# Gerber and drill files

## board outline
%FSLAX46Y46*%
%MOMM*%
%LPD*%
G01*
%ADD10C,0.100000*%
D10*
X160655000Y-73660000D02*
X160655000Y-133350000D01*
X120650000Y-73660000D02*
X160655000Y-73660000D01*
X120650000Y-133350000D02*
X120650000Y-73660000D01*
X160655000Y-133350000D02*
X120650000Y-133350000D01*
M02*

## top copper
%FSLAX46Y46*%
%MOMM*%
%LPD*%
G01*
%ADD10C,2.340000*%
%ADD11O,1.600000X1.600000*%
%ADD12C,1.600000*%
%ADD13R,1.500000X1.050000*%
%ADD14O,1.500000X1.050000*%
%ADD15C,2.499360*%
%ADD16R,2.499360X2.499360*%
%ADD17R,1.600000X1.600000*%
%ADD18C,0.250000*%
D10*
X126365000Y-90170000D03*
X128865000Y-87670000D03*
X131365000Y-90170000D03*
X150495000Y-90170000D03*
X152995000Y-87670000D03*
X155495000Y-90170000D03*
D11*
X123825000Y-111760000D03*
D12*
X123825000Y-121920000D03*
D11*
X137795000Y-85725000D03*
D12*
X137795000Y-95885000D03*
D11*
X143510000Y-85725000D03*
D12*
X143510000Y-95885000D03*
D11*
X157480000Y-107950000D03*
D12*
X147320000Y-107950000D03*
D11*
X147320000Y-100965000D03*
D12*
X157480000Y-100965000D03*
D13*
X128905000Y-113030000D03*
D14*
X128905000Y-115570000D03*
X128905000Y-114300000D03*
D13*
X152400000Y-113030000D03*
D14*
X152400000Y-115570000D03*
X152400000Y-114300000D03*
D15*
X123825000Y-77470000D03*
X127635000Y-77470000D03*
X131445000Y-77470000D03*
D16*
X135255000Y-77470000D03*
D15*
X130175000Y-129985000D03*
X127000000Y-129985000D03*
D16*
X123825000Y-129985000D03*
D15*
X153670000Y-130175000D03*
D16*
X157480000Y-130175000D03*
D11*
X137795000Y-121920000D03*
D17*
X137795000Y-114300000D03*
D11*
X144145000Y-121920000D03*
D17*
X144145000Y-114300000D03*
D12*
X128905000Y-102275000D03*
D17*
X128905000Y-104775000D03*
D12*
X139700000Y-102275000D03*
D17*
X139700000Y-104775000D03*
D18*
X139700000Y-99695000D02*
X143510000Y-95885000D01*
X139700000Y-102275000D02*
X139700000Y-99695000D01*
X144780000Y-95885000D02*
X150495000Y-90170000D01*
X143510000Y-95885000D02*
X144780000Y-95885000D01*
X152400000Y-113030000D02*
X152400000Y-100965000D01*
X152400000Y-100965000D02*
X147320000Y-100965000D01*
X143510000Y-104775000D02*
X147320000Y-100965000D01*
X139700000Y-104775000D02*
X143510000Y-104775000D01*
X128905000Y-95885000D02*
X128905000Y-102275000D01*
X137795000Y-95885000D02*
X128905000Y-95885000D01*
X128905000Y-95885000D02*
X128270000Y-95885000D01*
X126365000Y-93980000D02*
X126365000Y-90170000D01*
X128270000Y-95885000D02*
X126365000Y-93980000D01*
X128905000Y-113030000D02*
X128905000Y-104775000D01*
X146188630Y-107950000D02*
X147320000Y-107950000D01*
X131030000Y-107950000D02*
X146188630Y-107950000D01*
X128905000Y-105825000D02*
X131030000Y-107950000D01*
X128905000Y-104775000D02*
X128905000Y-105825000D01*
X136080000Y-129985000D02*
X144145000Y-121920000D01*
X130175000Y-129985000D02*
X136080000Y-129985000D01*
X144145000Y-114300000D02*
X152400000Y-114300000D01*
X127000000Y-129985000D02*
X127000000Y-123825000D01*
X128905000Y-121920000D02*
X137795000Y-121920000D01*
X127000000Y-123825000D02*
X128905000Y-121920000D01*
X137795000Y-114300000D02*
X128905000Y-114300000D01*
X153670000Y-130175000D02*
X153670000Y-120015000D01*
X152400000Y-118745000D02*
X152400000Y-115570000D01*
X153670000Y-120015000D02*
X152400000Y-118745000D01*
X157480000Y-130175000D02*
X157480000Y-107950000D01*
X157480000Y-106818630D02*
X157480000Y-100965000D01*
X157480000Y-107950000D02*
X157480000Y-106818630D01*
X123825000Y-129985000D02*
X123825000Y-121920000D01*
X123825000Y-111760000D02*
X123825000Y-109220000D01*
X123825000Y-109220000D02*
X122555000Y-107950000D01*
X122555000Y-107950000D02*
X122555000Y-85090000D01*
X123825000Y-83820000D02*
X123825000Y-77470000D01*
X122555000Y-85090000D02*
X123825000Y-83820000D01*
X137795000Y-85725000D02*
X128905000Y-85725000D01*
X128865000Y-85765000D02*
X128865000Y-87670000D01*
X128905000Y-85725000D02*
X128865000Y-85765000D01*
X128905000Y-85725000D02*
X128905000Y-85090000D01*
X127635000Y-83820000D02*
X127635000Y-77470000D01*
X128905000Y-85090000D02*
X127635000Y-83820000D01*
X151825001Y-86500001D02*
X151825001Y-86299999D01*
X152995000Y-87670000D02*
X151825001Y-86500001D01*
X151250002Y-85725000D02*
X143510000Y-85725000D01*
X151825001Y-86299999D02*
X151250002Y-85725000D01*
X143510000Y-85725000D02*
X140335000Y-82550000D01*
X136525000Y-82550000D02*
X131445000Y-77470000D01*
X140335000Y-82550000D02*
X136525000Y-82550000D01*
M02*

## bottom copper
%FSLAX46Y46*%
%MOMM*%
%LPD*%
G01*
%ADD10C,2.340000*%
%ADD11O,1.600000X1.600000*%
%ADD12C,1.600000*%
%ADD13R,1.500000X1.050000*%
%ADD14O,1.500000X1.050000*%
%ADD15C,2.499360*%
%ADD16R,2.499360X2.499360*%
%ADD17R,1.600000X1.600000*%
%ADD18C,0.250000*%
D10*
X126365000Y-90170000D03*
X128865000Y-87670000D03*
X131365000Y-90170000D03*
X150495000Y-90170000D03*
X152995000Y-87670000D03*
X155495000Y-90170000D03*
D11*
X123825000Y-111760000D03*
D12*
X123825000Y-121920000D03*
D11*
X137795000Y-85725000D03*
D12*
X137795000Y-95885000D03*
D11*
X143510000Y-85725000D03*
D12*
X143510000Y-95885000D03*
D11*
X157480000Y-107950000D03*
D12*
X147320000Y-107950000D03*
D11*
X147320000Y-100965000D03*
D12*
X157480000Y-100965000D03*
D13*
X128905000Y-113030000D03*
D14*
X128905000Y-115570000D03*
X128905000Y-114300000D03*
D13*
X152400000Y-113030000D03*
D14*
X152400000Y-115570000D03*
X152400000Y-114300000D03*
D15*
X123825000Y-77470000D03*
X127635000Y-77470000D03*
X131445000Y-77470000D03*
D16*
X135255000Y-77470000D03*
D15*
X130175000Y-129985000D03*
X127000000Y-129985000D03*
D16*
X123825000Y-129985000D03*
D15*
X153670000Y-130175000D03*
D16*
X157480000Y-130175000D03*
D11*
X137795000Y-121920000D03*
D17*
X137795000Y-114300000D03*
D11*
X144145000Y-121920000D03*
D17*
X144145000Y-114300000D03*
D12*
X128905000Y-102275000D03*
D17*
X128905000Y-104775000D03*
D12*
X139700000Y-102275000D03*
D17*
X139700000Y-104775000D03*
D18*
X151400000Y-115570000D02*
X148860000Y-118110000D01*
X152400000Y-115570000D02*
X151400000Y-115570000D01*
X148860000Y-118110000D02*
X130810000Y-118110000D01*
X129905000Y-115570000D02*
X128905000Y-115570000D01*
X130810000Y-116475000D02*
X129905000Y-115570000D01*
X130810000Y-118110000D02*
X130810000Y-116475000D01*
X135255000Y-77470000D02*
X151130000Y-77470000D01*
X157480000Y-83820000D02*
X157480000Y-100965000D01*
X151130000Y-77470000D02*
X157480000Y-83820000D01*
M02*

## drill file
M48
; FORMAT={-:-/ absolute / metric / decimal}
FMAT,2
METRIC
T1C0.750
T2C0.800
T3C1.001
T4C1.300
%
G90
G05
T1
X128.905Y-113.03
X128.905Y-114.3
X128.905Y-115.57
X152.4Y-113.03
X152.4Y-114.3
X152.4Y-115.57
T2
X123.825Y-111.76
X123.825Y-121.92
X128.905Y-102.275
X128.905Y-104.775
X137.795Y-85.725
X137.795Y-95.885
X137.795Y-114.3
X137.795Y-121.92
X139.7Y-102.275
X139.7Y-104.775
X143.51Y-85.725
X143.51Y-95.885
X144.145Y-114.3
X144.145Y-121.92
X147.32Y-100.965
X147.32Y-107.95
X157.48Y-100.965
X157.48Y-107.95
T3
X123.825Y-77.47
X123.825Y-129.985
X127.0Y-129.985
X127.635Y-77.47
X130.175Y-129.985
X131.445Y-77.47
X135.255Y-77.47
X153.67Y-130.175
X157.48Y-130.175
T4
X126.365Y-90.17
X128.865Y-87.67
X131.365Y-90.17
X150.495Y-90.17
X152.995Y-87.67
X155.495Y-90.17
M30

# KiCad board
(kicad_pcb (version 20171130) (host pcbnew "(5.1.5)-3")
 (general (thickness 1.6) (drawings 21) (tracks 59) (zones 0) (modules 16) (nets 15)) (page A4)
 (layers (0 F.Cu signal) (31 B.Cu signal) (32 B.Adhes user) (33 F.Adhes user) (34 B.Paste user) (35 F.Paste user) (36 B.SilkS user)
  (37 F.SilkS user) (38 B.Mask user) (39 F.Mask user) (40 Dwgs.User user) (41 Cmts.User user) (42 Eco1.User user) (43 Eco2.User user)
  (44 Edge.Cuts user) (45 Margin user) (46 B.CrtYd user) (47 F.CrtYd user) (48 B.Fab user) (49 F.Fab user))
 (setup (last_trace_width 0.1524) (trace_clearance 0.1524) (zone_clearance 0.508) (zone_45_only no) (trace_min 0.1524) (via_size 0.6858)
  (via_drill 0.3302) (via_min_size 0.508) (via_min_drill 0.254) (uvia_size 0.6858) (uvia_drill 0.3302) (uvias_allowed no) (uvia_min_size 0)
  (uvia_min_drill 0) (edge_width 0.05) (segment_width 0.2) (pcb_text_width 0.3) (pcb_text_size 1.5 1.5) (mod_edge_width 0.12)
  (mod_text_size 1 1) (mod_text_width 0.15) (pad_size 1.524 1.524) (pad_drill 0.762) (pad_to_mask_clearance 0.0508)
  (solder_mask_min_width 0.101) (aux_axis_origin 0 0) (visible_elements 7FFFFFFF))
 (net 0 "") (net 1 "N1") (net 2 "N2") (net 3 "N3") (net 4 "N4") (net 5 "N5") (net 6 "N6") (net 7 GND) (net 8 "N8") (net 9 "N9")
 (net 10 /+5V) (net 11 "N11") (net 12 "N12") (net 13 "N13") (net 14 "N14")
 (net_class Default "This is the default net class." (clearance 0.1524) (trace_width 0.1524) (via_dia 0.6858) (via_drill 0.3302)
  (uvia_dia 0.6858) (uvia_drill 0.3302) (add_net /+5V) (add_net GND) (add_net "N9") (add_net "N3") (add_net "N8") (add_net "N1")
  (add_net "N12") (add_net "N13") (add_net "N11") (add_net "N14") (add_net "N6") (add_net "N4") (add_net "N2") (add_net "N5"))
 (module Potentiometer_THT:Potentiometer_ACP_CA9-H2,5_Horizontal (layer F.Cu) (at 126.365 90.17 90)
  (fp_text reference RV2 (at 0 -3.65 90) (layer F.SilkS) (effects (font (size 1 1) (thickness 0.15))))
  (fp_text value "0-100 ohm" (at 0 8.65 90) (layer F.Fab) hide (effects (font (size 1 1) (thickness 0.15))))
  (pad 1 thru_hole circle (at 0 0 90) (size 2.34 2.34) (drill 1.3) (layers *.Cu *.Mask) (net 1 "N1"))
  (pad 2 thru_hole circle (at 2.5 2.5 90) (size 2.34 2.34) (drill 1.3) (layers *.Cu *.Mask) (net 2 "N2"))
  (pad 3 thru_hole circle (at 0 5 90) (size 2.34 2.34) (drill 1.3) (layers *.Cu *.Mask)))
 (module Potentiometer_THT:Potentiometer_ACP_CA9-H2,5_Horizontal (layer F.Cu) (at 150.495 90.17 90)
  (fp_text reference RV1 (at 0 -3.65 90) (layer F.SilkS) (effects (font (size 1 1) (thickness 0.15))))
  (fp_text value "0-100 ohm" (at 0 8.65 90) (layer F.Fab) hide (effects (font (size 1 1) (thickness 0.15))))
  (pad 1 thru_hole circle (at 0 0 90) (size 2.34 2.34) (drill 1.3) (layers *.Cu *.Mask) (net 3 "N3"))
  (pad 2 thru_hole circle (at 2.5 2.5 90) (size 2.34 2.34) (drill 1.3) (layers *.Cu *.Mask) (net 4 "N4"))
  (pad 3 thru_hole circle (at 0 5 90) (size 2.34 2.34) (drill 1.3) (layers *.Cu *.Mask)))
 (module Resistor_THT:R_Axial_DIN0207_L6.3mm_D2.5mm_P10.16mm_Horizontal (layer F.Cu) (at 123.825 121.92 90)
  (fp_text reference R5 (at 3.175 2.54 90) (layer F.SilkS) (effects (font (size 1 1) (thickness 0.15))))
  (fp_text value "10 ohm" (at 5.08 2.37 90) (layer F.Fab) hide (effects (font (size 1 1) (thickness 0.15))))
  (pad 2 thru_hole oval (at 10.16 0 90) (size 1.6 1.6) (drill 0.8) (layers *.Cu *.Mask) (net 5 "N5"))
  (pad 1 thru_hole circle (at 0 0 90) (size 1.6 1.6) (drill 0.8) (layers *.Cu *.Mask) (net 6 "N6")))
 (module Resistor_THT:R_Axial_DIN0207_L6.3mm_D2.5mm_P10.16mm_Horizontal (layer F.Cu) (at 137.795 95.885 90)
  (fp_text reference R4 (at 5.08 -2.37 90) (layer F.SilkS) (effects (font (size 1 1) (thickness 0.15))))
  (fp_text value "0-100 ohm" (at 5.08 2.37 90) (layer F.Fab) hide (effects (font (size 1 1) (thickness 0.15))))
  (pad 2 thru_hole oval (at 10.16 0 90) (size 1.6 1.6) (drill 0.8) (layers *.Cu *.Mask) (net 2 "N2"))
  (pad 1 thru_hole circle (at 0 0 90) (size 1.6 1.6) (drill 0.8) (layers *.Cu *.Mask) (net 1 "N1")))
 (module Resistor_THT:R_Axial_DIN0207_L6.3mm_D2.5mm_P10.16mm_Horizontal (layer F.Cu) (at 143.51 95.885 90)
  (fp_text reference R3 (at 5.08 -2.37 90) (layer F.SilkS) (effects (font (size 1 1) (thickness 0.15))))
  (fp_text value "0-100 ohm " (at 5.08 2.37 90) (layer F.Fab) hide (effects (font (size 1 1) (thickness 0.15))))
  (pad 2 thru_hole oval (at 10.16 0 90) (size 1.6 1.6) (drill 0.8) (layers *.Cu *.Mask) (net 4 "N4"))
  (pad 1 thru_hole circle (at 0 0 90) (size 1.6 1.6) (drill 0.8) (layers *.Cu *.Mask) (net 3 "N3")))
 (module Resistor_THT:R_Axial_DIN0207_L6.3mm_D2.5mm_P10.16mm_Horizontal (layer F.Cu) (at 147.32 107.95)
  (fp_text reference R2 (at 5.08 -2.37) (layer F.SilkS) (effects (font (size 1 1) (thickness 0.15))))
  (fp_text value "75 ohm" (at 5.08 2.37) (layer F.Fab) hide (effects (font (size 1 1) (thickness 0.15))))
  (pad 2 thru_hole oval (at 10.16 0) (size 1.6 1.6) (drill 0.8) (layers *.Cu *.Mask) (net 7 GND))
  (pad 1 thru_hole circle (at 0 0) (size 1.6 1.6) (drill 0.8) (layers *.Cu *.Mask) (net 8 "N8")))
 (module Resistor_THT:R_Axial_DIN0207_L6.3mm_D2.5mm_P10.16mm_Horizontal (layer F.Cu) (at 157.48 100.965 180)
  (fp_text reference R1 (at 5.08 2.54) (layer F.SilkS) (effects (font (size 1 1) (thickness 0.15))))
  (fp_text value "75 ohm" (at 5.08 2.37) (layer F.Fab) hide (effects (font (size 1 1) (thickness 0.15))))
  (pad 2 thru_hole oval (at 10.16 0 180) (size 1.6 1.6) (drill 0.8) (layers *.Cu *.Mask) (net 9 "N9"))
  (pad 1 thru_hole circle (at 0 0 180) (size 1.6 1.6) (drill 0.8) (layers *.Cu *.Mask) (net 7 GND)))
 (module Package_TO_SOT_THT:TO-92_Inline (layer F.Cu) (at 128.905 113.03 270)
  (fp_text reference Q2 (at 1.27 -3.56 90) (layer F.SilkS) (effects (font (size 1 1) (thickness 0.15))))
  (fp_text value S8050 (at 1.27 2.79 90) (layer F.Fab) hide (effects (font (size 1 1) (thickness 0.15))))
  (pad 1 thru_hole rect (at 0 0 270) (size 1.05 1.5) (drill 0.75) (layers *.Cu *.Mask) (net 8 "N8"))
  (pad 3 thru_hole oval (at 2.54 0 270) (size 1.05 1.5) (drill 0.75) (layers *.Cu *.Mask) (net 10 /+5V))
  (pad 2 thru_hole oval (at 1.27 0 270) (size 1.05 1.5) (drill 0.75) (layers *.Cu *.Mask) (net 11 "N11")))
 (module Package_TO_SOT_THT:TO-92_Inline (layer F.Cu) (at 152.4 113.03 270)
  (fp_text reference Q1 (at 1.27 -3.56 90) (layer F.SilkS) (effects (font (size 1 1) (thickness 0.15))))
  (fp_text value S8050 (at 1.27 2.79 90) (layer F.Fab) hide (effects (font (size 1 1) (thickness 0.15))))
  (pad 1 thru_hole rect (at 0 0 270) (size 1.05 1.5) (drill 0.75) (layers *.Cu *.Mask) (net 9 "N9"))
  (pad 3 thru_hole oval (at 2.54 0 270) (size 1.05 1.5) (drill 0.75) (layers *.Cu *.Mask) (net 10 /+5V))
  (pad 2 thru_hole oval (at 1.27 0 270) (size 1.05 1.5) (drill 0.75) (layers *.Cu *.Mask) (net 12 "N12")))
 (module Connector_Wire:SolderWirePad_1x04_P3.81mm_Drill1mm (layer F.Cu) (at 135.255 77.47 180)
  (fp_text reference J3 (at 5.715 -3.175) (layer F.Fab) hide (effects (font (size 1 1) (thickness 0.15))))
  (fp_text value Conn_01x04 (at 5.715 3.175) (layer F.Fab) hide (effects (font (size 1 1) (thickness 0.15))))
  (pad 4 thru_hole circle (at 11.43 0 180) (size 2.49936 2.49936) (drill 1.00076) (layers *.Cu *.Mask) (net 5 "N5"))
  (pad 3 thru_hole circle (at 7.62 0 180) (size 2.49936 2.49936) (drill 1.00076) (layers *.Cu *.Mask) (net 2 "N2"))
  (pad 2 thru_hole circle (at 3.81 0 180) (size 2.49936 2.49936) (drill 1.00076) (layers *.Cu *.Mask) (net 4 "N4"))
  (pad 1 thru_hole rect (at 0 0 180) (size 2.49936 2.49936) (drill 1.00076) (layers *.Cu *.Mask) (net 7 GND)))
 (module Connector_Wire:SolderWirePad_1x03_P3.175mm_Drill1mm (layer F.Cu) (at 123.825 129.985)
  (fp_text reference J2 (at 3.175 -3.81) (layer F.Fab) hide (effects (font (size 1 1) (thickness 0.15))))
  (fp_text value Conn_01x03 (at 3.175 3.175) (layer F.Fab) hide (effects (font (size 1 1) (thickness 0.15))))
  (pad 3 thru_hole circle (at 6.35 0) (size 2.49936 2.49936) (drill 1.00076) (layers *.Cu *.Mask) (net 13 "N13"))
  (pad 2 thru_hole circle (at 3.175 0) (size 2.49936 2.49936) (drill 1.00076) (layers *.Cu *.Mask) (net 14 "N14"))
  (pad 1 thru_hole rect (at 0 0) (size 2.49936 2.49936) (drill 1.00076) (layers *.Cu *.Mask) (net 6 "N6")))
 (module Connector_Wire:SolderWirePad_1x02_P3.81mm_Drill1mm (layer F.Cu) (at 157.48 130.175 180)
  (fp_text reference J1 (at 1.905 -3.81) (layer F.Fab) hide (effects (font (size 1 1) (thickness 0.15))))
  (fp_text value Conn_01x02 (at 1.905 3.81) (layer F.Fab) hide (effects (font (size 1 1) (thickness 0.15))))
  (pad 2 thru_hole circle (at 3.81 0 180) (size 2.49936 2.49936) (drill 1.00076) (layers *.Cu *.Mask) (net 10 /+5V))
  (pad 1 thru_hole rect (at 0 0 180) (size 2.49936 2.49936) (drill 1.00076) (layers *.Cu *.Mask) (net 7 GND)))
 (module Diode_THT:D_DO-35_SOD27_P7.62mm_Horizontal (layer F.Cu) (at 137.795 114.3 270)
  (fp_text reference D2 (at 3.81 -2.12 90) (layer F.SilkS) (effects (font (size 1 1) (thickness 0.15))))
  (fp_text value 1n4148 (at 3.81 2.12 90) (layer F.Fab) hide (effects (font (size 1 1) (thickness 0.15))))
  (pad 2 thru_hole oval (at 7.62 0 270) (size 1.6 1.6) (drill 0.8) (layers *.Cu *.Mask) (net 14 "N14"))
  (pad 1 thru_hole rect (at 0 0 270) (size 1.6 1.6) (drill 0.8) (layers *.Cu *.Mask) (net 11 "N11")))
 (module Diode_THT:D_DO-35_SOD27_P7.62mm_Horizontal (layer F.Cu) (at 144.145 114.3 270)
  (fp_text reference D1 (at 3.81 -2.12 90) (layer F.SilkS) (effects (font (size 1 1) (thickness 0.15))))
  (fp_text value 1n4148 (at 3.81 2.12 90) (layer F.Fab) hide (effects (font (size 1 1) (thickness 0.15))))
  (pad 2 thru_hole oval (at 7.62 0 270) (size 1.6 1.6) (drill 0.8) (layers *.Cu *.Mask) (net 13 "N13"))
  (pad 1 thru_hole rect (at 0 0 270) (size 1.6 1.6) (drill 0.8) (layers *.Cu *.Mask) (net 12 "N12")))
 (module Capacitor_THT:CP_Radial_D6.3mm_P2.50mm (layer F.Cu) (at 128.905 104.775 90)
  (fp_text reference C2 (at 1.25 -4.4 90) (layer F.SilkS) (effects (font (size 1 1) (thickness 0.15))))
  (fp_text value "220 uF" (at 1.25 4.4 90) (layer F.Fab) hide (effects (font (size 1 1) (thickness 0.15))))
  (pad 2 thru_hole circle (at 2.5 0 90) (size 1.6 1.6) (drill 0.8) (layers *.Cu *.Mask) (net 1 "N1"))
  (pad 1 thru_hole rect (at 0 0 90) (size 1.6 1.6) (drill 0.8) (layers *.Cu *.Mask) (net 8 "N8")))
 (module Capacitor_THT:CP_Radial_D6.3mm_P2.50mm (layer F.Cu) (at 139.7 104.775 90)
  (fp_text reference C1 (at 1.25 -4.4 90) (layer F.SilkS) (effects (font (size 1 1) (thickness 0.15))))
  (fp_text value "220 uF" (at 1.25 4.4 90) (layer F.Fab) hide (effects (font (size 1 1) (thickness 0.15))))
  (pad 2 thru_hole circle (at 2.5 0 90) (size 1.6 1.6) (drill 0.8) (layers *.Cu *.Mask) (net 3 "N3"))
  (pad 1 thru_hole rect (at 0 0 90) (size 1.6 1.6) (drill 0.8) (layers *.Cu *.Mask) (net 9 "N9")))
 (gr_line (start 160.655 73.66) (end 160.655 133.35) (layer Edge.Cuts) (width 0.1))
 (gr_line (start 120.65 73.66) (end 160.655 73.66) (layer Edge.Cuts) (width 0.1))
 (gr_line (start 120.65 133.35) (end 120.65 73.66) (layer Edge.Cuts) (width 0.1))
 (gr_line (start 160.655 133.35) (end 120.65 133.35) (layer Edge.Cuts) (width 0.1))
 (segment (start 139.7 99.695) (end 143.51 95.885) (width 0.25) (layer F.Cu) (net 3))
 (segment (start 139.7 102.275) (end 139.7 99.695) (width 0.25) (layer F.Cu) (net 3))
 (segment (start 144.78 95.885) (end 150.495 90.17) (width 0.25) (layer F.Cu) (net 3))
 (segment (start 143.51 95.885) (end 144.78 95.885) (width 0.25) (layer F.Cu) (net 3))
 (segment (start 152.4 113.03) (end 152.4 100.965) (width 0.25) (layer F.Cu) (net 9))
 (segment (start 152.4 100.965) (end 147.32 100.965) (width 0.25) (layer F.Cu) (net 9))
 (segment (start 143.51 104.775) (end 147.32 100.965) (width 0.25) (layer F.Cu) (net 9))
 (segment (start 139.7 104.775) (end 143.51 104.775) (width 0.25) (layer F.Cu) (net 9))
 (segment (start 128.905 95.885) (end 128.905 102.275) (width 0.25) (layer F.Cu) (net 1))
 (segment (start 137.795 95.885) (end 128.905 95.885) (width 0.25) (layer F.Cu) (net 1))
 (segment (start 128.905 95.885) (end 128.27 95.885) (width 0.25) (layer F.Cu) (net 1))
 (segment (start 126.365 93.98) (end 126.365 90.17) (width 0.25) (layer F.Cu) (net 1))
 (segment (start 128.27 95.885) (end 126.365 93.98) (width 0.25) (layer F.Cu) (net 1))
 (segment (start 128.905 113.03) (end 128.905 104.775) (width 0.25) (layer F.Cu) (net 8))
 (segment (start 146.18863 107.95) (end 147.32 107.95) (width 0.25) (layer F.Cu) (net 8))
 (segment (start 131.03 107.95) (end 146.18863 107.95) (width 0.25) (layer F.Cu) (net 8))
 (segment (start 128.905 105.825) (end 131.03 107.95) (width 0.25) (layer F.Cu) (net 8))
 (segment (start 128.905 104.775) (end 128.905 105.825) (width 0.25) (layer F.Cu) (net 8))
 (segment (start 136.08 129.985) (end 144.145 121.92) (width 0.25) (layer F.Cu) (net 13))
 (segment (start 130.175 129.985) (end 136.08 129.985) (width 0.25) (layer F.Cu) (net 13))
 (segment (start 144.145 114.3) (end 152.4 114.3) (width 0.25) (layer F.Cu) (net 12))
 (segment (start 127 129.985) (end 127 123.825) (width 0.25) (layer F.Cu) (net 14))
 (segment (start 128.905 121.92) (end 137.795 121.92) (width 0.25) (layer F.Cu) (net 14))
 (segment (start 127 123.825) (end 128.905 121.92) (width 0.25) (layer F.Cu) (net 14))
 (segment (start 137.795 114.3) (end 128.905 114.3) (width 0.25) (layer F.Cu) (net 11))
 (segment (start 153.67 130.175) (end 153.67 120.015) (width 0.25) (layer F.Cu) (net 10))
 (segment (start 152.4 118.745) (end 152.4 115.57) (width 0.25) (layer F.Cu) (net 10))
 (segment (start 153.67 120.015) (end 152.4 118.745) (width 0.25) (layer F.Cu) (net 10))
 (segment (start 151.4 115.57) (end 148.86 118.11) (width 0.25) (layer B.Cu) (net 10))
 (segment (start 152.4 115.57) (end 151.4 115.57) (width 0.25) (layer B.Cu) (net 10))
 (segment (start 148.86 118.11) (end 130.81 118.11) (width 0.25) (layer B.Cu) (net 10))
 (segment (start 129.905 115.57) (end 128.905 115.57) (width 0.25) (layer B.Cu) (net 10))
 (segment (start 130.81 116.475) (end 129.905 115.57) (width 0.25) (layer B.Cu) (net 10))
 (segment (start 130.81 118.11) (end 130.81 116.475) (width 0.25) (layer B.Cu) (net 10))
 (segment (start 157.48 130.175) (end 157.48 107.95) (width 0.25) (layer F.Cu) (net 7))
 (segment (start 157.48 106.81863) (end 157.48 100.965) (width 0.25) (layer F.Cu) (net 7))
 (segment (start 157.48 107.95) (end 157.48 106.81863) (width 0.25) (layer F.Cu) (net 7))
 (segment (start 135.255 77.47) (end 151.13 77.47) (width 0.25) (layer B.Cu) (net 7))
 (segment (start 157.48 83.82) (end 157.48 100.965) (width 0.25) (layer B.Cu) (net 7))
 (segment (start 151.13 77.47) (end 157.48 83.82) (width 0.25) (layer B.Cu) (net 7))
 (segment (start 123.825 129.985) (end 123.825 121.92) (width 0.25) (layer F.Cu) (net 6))
 (segment (start 123.825 111.76) (end 123.825 109.22) (width 0.25) (layer F.Cu) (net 5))
 (segment (start 123.825 109.22) (end 122.555 107.95) (width 0.25) (layer F.Cu) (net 5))
 (segment (start 122.555 107.95) (end 122.555 85.09) (width 0.25) (layer F.Cu) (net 5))
 (segment (start 123.825 83.82) (end 123.825 77.47) (width 0.25) (layer F.Cu) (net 5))
 (segment (start 122.555 85.09) (end 123.825 83.82) (width 0.25) (layer F.Cu) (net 5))
 (segment (start 137.795 85.725) (end 128.905 85.725) (width 0.25) (layer F.Cu) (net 2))
 (segment (start 128.865 85.765) (end 128.865 87.67) (width 0.25) (layer F.Cu) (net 2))
 (segment (start 128.905 85.725) (end 128.865 85.765) (width 0.25) (layer F.Cu) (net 2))
 (segment (start 128.905 85.725) (end 128.905 85.09) (width 0.25) (layer F.Cu) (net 2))
 (segment (start 127.635 83.82) (end 127.635 77.47) (width 0.25) (layer F.Cu) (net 2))
 (segment (start 128.905 85.09) (end 127.635 83.82) (width 0.25) (layer F.Cu) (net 2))
 (segment (start 151.825001 86.500001) (end 151.825001 86.299999) (width 0.25) (layer F.Cu) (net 4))
 (segment (start 152.995 87.67) (end 151.825001 86.500001) (width 0.25) (layer F.Cu) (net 4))
 (segment (start 151.250002 85.725) (end 143.51 85.725) (width 0.25) (layer F.Cu) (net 4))
 (segment (start 151.825001 86.299999) (end 151.250002 85.725) (width 0.25) (layer F.Cu) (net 4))
 (segment (start 143.51 85.725) (end 140.335 82.55) (width 0.25) (layer F.Cu) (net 4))
 (segment (start 136.525 82.55) (end 131.445 77.47) (width 0.25) (layer F.Cu) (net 4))
 (segment (start 140.335 82.55) (end 136.525 82.55) (width 0.25) (layer F.Cu) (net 4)))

